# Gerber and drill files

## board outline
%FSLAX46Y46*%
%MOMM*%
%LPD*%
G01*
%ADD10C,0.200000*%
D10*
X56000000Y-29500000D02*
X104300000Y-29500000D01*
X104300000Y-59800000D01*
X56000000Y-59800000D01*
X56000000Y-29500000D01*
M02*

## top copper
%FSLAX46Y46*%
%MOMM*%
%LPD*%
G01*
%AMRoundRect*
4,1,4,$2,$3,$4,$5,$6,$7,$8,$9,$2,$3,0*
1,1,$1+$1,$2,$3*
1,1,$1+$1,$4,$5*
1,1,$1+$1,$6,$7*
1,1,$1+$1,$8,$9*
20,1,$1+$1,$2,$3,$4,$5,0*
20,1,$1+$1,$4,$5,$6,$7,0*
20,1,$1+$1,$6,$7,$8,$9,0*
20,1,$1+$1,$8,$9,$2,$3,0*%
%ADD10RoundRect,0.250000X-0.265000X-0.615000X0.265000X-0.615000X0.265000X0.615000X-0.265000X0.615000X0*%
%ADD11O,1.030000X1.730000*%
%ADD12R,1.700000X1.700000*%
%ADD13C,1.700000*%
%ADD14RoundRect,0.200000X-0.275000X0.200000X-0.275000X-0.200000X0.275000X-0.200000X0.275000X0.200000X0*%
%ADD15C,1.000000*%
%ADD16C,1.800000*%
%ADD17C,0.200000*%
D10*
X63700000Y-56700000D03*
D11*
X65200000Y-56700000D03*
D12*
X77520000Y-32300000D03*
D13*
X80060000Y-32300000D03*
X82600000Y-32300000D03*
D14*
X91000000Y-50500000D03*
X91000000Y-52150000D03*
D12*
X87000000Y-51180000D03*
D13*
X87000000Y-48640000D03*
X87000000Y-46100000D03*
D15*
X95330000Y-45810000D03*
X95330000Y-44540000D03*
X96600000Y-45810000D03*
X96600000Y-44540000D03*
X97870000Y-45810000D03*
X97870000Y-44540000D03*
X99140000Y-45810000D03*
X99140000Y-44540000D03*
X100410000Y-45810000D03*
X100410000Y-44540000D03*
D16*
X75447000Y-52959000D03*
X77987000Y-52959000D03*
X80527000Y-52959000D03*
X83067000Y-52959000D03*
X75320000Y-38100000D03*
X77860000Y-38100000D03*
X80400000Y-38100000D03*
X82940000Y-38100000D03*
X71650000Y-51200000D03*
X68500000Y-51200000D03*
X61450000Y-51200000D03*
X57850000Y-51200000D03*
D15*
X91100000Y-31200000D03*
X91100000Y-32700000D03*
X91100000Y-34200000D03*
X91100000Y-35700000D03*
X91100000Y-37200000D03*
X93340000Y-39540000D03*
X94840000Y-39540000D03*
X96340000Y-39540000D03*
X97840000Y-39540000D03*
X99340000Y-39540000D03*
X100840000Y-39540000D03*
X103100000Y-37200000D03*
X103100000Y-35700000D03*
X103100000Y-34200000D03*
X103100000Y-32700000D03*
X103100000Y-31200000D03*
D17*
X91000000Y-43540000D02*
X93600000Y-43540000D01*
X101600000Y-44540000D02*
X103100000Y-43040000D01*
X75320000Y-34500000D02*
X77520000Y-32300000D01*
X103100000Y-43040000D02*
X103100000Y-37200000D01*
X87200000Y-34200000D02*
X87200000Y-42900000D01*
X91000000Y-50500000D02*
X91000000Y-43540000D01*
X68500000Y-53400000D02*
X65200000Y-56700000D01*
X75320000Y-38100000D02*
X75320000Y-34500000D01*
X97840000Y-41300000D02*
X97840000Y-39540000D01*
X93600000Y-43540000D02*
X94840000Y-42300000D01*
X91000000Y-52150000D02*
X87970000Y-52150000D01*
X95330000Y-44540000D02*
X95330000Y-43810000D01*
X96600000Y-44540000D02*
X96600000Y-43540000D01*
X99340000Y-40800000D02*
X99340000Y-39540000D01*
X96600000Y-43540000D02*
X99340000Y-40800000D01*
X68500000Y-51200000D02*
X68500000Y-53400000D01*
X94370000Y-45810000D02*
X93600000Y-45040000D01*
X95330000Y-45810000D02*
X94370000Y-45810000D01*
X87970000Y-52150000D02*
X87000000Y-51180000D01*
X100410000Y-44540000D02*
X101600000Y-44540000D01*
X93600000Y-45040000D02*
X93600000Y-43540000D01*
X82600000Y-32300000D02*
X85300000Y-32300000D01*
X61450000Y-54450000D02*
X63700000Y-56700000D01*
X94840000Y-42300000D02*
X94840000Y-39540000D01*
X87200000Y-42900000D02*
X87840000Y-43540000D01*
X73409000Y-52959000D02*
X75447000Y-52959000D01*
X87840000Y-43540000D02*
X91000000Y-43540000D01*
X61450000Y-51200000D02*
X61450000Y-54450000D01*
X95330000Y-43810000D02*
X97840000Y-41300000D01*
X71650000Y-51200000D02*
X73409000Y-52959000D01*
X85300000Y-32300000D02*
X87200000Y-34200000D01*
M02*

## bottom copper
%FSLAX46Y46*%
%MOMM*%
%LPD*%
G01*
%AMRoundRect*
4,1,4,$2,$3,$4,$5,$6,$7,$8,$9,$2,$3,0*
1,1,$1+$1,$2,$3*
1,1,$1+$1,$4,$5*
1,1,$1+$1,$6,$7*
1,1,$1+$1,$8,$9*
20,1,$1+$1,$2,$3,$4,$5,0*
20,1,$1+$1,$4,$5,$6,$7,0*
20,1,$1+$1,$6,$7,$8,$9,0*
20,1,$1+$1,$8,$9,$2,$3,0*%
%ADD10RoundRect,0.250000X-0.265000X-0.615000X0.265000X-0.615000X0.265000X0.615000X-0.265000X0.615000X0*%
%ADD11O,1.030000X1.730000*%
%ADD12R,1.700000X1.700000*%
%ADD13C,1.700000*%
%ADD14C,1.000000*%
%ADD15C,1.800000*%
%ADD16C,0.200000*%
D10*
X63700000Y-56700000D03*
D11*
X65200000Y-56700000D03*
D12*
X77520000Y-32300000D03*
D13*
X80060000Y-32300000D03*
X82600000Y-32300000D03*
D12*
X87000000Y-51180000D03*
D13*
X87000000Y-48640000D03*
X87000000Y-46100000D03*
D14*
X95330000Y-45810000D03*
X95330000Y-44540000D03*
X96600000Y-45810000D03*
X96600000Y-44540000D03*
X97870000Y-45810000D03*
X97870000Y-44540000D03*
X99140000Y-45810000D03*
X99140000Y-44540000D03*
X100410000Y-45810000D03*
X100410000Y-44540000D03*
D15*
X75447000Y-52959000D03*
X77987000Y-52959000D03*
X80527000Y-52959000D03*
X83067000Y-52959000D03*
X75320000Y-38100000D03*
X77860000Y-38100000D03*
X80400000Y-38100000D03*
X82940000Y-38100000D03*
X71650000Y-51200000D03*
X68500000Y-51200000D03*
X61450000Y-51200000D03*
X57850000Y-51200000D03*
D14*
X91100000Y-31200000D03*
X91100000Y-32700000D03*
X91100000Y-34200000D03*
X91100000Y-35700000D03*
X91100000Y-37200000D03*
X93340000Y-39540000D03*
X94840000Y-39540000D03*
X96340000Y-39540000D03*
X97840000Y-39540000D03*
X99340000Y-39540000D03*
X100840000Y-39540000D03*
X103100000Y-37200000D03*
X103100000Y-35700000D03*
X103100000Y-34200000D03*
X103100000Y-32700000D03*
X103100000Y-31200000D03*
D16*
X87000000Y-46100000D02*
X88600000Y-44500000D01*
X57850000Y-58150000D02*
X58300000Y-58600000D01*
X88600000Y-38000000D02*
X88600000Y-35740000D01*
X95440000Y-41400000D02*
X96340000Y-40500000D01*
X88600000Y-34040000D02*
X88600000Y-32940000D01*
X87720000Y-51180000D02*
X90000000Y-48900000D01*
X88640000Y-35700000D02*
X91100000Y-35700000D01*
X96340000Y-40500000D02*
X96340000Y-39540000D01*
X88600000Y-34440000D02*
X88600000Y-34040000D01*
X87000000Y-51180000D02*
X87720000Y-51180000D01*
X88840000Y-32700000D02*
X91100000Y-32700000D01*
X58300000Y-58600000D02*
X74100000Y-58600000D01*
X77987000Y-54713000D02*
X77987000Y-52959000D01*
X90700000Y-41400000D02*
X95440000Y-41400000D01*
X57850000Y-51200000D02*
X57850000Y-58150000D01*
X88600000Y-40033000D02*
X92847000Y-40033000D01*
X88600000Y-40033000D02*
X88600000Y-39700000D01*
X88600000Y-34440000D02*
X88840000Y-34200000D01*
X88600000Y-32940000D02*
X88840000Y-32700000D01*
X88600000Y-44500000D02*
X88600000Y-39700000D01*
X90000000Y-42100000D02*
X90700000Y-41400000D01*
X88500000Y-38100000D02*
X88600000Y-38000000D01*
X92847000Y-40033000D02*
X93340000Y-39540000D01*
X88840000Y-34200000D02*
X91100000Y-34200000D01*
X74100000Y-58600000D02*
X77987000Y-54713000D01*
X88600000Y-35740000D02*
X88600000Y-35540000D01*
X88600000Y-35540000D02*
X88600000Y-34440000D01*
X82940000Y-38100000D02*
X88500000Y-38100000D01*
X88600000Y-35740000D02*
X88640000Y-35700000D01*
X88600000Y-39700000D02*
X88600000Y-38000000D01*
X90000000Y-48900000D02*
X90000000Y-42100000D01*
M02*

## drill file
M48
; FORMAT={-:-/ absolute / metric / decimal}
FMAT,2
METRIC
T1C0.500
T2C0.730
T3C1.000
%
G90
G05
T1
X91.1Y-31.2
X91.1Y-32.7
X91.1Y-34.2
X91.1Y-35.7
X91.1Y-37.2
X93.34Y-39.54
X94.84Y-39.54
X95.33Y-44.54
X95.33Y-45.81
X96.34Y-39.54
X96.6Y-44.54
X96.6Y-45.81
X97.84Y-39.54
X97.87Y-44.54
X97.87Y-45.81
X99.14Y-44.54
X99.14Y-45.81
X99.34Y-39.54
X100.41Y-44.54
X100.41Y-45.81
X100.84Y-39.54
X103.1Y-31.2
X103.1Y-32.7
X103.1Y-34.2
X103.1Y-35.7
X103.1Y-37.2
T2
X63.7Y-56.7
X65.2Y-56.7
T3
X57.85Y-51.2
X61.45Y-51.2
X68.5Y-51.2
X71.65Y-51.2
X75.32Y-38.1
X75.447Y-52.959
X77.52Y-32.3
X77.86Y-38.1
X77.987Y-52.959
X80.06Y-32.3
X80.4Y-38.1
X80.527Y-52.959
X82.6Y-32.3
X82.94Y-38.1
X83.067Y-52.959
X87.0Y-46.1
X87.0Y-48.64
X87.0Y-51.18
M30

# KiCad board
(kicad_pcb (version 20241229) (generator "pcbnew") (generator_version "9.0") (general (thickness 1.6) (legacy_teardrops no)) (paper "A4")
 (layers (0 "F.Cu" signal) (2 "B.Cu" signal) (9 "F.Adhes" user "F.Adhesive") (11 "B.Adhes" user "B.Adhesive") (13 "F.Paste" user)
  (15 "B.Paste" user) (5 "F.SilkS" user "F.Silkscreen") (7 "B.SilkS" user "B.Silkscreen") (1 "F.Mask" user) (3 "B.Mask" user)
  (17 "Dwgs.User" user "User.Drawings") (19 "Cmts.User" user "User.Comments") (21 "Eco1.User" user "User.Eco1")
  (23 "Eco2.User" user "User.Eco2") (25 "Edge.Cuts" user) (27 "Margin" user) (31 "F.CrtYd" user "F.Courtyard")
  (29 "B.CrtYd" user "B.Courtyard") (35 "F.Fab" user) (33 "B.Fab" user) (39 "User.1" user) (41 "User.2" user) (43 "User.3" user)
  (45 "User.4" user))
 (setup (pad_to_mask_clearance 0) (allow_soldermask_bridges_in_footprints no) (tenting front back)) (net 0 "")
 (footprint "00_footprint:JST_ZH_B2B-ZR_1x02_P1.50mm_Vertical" (layer "F.Cu") (at 63.7 56.7)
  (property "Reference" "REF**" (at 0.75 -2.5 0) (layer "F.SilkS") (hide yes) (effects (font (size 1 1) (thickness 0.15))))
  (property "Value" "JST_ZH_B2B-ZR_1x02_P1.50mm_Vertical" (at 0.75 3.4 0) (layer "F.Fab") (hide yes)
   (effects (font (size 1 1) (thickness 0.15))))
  (pad "1" thru_hole roundrect (at 0 0) (size 1.03 1.73) (drill 0.73) (layers "*.Cu" "*.Mask") (remove_unused_layers no)
   (roundrect_rratio 0.242718))
  (pad "2" thru_hole oval (at 1.5 0) (size 1.03 1.73) (drill 0.73) (layers "*.Cu" "*.Mask") (remove_unused_layers no)))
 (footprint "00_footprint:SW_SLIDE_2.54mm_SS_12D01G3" (layer "F.Cu") (at 77.52 32.3 90)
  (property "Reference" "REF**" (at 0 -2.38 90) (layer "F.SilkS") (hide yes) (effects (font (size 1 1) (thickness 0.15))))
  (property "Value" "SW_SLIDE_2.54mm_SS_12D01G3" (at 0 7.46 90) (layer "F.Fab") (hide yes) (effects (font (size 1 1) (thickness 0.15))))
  (pad "1" thru_hole rect (at 0 0 90) (size 1.7 1.7) (drill 1) (layers "*.Cu" "*.Mask") (remove_unused_layers no))
  (pad "2" thru_hole circle (at 0 2.54 90) (size 1.7 1.7) (drill 1) (layers "*.Cu" "*.Mask") (remove_unused_layers no))
  (pad "3" thru_hole circle (at 0 5.08 90) (size 1.7 1.7) (drill 1) (layers "*.Cu" "*.Mask") (remove_unused_layers no)))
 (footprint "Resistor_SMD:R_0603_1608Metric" (layer "F.Cu") (at 91 51.325 -90)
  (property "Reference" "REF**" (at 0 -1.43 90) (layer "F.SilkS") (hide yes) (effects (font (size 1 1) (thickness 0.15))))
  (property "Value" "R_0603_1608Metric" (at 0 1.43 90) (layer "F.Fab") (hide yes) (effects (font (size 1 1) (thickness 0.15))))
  (pad "1" smd roundrect (at -0.825 0 270) (size 0.8 0.95) (layers "F.Cu" "F.Mask" "F.Paste") (roundrect_rratio 0.25))
  (pad "2" smd roundrect (at 0.825 0 270) (size 0.8 0.95) (layers "F.Cu" "F.Mask" "F.Paste") (roundrect_rratio 0.25)))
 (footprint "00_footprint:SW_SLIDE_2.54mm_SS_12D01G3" (layer "F.Cu") (at 87 51.18 180)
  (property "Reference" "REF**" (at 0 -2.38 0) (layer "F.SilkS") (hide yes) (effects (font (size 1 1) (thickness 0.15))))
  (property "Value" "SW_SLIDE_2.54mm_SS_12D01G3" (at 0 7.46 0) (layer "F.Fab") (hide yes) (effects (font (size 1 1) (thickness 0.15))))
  (pad "1" thru_hole rect (at 0 0 180) (size 1.7 1.7) (drill 1) (layers "*.Cu" "*.Mask") (remove_unused_layers no))
  (pad "2" thru_hole circle (at 0 2.54 180) (size 1.7 1.7) (drill 1) (layers "*.Cu" "*.Mask") (remove_unused_layers no))
  (pad "3" thru_hole circle (at 0 5.08 180) (size 1.7 1.7) (drill 1) (layers "*.Cu" "*.Mask") (remove_unused_layers no)))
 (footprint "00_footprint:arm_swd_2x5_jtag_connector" (layer "F.Cu") (at 97.87 45.81 180)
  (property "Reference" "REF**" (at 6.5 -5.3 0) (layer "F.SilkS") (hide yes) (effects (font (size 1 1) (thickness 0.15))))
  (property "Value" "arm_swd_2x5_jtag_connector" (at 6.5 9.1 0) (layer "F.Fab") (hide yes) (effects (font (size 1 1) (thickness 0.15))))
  (pad "1" thru_hole circle (at 2.54 0 270) (size 1 1) (drill 0.5) (layers "*.Cu" "*.Mask") (remove_unused_layers no))
  (pad "2" thru_hole circle (at 2.54 1.27 270) (size 1 1) (drill 0.5) (layers "*.Cu" "*.Mask") (remove_unused_layers no))
  (pad "3" thru_hole circle (at 1.27 0 270) (size 1 1) (drill 0.5) (layers "*.Cu" "*.Mask") (remove_unused_layers no))
  (pad "4" thru_hole circle (at 1.27 1.27 270) (size 1 1) (drill 0.5) (layers "*.Cu" "*.Mask") (remove_unused_layers no))
  (pad "5" thru_hole circle (at 0 0 270) (size 1 1) (drill 0.5) (layers "*.Cu" "*.Mask") (remove_unused_layers no))
  (pad "6" thru_hole circle (at 0 1.27 270) (size 1 1) (drill 0.5) (layers "*.Cu" "*.Mask") (remove_unused_layers no))
  (pad "7" thru_hole circle (at -1.27 0 270) (size 1 1) (drill 0.5) (layers "*.Cu" "*.Mask") (remove_unused_layers no))
  (pad "8" thru_hole circle (at -1.27 1.27 270) (size 1 1) (drill 0.5) (layers "*.Cu" "*.Mask") (remove_unused_layers no))
  (pad "9" thru_hole circle (at -2.54 0 270) (size 1 1) (drill 0.5) (layers "*.Cu" "*.Mask") (remove_unused_layers no))
  (pad "10" thru_hole circle (at -2.54 1.27 270) (size 1 1) (drill 0.5) (layers "*.Cu" "*.Mask") (remove_unused_layers no)))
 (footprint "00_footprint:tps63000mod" (layer "F.Cu") (at 79.257 45.593 90)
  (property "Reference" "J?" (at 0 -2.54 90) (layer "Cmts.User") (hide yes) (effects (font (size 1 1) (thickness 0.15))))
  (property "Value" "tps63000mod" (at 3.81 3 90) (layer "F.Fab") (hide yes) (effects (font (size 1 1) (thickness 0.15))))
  (pad "1" thru_hole circle (at -7.366 -3.81 90) (size 1.8 1.8) (drill 1) (layers "*.Cu" "*.Mask") (remove_unused_layers no))
  (pad "2" thru_hole circle (at -7.366 -1.27 90) (size 1.8 1.8) (drill 1) (layers "*.Cu" "*.Mask") (remove_unused_layers no))
  (pad "3" thru_hole circle (at -7.366 1.27 90) (size 1.8 1.8) (drill 1) (layers "*.Cu" "*.Mask") (remove_unused_layers no))
  (pad "4" thru_hole circle (at -7.366 3.81 90) (size 1.8 1.8) (drill 1) (layers "*.Cu" "*.Mask") (remove_unused_layers no))
  (pad "5" thru_hole circle (at 7.493 -3.937 90) (size 1.8 1.8) (drill 1) (layers "*.Cu" "*.Mask") (remove_unused_layers no))
  (pad "6" thru_hole circle (at 7.493 -1.397 90) (size 1.8 1.8) (drill 1) (layers "*.Cu" "*.Mask") (remove_unused_layers no))
  (pad "7" thru_hole circle (at 7.493 1.143 90) (size 1.8 1.8) (drill 1) (layers "*.Cu" "*.Mask") (remove_unused_layers no))
  (pad "8" thru_hole circle (at 7.493 3.683 90) (size 1.8 1.8) (drill 1) (layers "*.Cu" "*.Mask") (remove_unused_layers no)))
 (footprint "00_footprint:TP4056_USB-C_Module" (layer "F.Cu") (at 64.4 42 -90)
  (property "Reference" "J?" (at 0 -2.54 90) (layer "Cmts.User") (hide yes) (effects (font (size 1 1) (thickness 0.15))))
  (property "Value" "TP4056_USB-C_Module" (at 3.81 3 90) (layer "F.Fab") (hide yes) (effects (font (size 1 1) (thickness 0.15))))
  (pad "1" thru_hole circle (at 9.2 -7.25 270) (size 1.8 1.8) (drill 1) (layers "*.Cu" "*.Mask") (remove_unused_layers no))
  (pad "2" thru_hole circle (at 9.2 -4.1 270) (size 1.8 1.8) (drill 1) (layers "*.Cu" "*.Mask") (remove_unused_layers no))
  (pad "3" thru_hole circle (at 9.2 2.95 270) (size 1.8 1.8) (drill 1) (layers "*.Cu" "*.Mask") (remove_unused_layers no))
  (pad "4" thru_hole circle (at 9.2 6.55 270) (size 1.8 1.8) (drill 1) (layers "*.Cu" "*.Mask") (remove_unused_layers no)))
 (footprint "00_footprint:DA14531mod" (layer "F.Cu") (at 97.1 34.54)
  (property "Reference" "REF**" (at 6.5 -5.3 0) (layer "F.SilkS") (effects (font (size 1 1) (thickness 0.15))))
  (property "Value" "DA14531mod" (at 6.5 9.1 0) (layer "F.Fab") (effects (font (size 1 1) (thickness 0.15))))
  (pad "J1" thru_hole circle (at -6 -3.34 90) (size 1 1) (drill 0.5) (layers "*.Cu" "*.Mask") (remove_unused_layers no))
  (pad "J2" thru_hole circle (at -6 -1.84 90) (size 1 1) (drill 0.5) (layers "*.Cu" "*.Mask") (remove_unused_layers no))
  (pad "J3" thru_hole circle (at -6 -0.34 90) (size 1 1) (drill 0.5) (layers "*.Cu" "*.Mask") (remove_unused_layers no))
  (pad "J4" thru_hole circle (at -6 1.16 90) (size 1 1) (drill 0.5) (layers "*.Cu" "*.Mask") (remove_unused_layers no))
  (pad "J5" thru_hole circle (at -6 2.66 90) (size 1 1) (drill 0.5) (layers "*.Cu" "*.Mask") (remove_unused_layers no))
  (pad "J6" thru_hole circle (at -3.76 5 90) (size 1 1) (drill 0.5) (layers "*.Cu" "*.Mask") (remove_unused_layers no))
  (pad "J7" thru_hole circle (at -2.26 5 90) (size 1 1) (drill 0.5) (layers "*.Cu" "*.Mask") (remove_unused_layers no))
  (pad "J8" thru_hole circle (at -0.76 5 90) (size 1 1) (drill 0.5) (layers "*.Cu" "*.Mask") (remove_unused_layers no))
  (pad "J9" thru_hole circle (at 0.74 5 90) (size 1 1) (drill 0.5) (layers "*.Cu" "*.Mask") (remove_unused_layers no))
  (pad "J10" thru_hole circle (at 2.24 5 90) (size 1 1) (drill 0.5) (layers "*.Cu" "*.Mask") (remove_unused_layers no))
  (pad "J11" thru_hole circle (at 3.74 5 90) (size 1 1) (drill 0.5) (layers "*.Cu" "*.Mask") (remove_unused_layers no))
  (pad "J12" thru_hole circle (at 6 2.66 90) (size 1 1) (drill 0.5) (layers "*.Cu" "*.Mask") (remove_unused_layers no))
  (pad "J13" thru_hole circle (at 6 1.16 90) (size 1 1) (drill 0.5) (layers "*.Cu" "*.Mask") (remove_unused_layers no))
  (pad "J14" thru_hole circle (at 6 -0.34 90) (size 1 1) (drill 0.5) (layers "*.Cu" "*.Mask") (remove_unused_layers no))
  (pad "J15" thru_hole circle (at 6 -1.84 90) (size 1 1) (drill 0.5) (layers "*.Cu" "*.Mask") (remove_unused_layers no))
  (pad "J16" thru_hole circle (at 6 -3.34 90) (size 1 1) (drill 0.5) (layers "*.Cu" "*.Mask") (remove_unused_layers no)))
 (gr_rect (start 56 29.5) (end 104.3 59.8) (stroke (width 0.2) (type solid)) (fill no) (layer "Edge.Cuts"))
 (segment (start 91 43.54) (end 93.6 43.54) (width 0.2) (layer "F.Cu") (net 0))
 (segment (start 101.6 44.54) (end 103.1 43.04) (width 0.2) (layer "F.Cu") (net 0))
 (segment (start 75.32 34.5) (end 77.52 32.3) (width 0.2) (layer "F.Cu") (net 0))
 (segment (start 103.1 43.04) (end 103.1 37.2) (width 0.2) (layer "F.Cu") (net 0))
 (segment (start 87.2 34.2) (end 87.2 42.9) (width 0.2) (layer "F.Cu") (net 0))
 (segment (start 91 50.5) (end 91 43.54) (width 0.2) (layer "F.Cu") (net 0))
 (segment (start 68.5 53.4) (end 65.2 56.7) (width 0.2) (layer "F.Cu") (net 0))
 (segment (start 75.32 38.1) (end 75.32 34.5) (width 0.2) (layer "F.Cu") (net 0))
 (segment (start 97.84 41.3) (end 97.84 39.54) (width 0.2) (layer "F.Cu") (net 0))
 (segment (start 93.6 43.54) (end 94.84 42.3) (width 0.2) (layer "F.Cu") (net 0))
 (segment (start 91 52.15) (end 87.97 52.15) (width 0.2) (layer "F.Cu") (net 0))
 (segment (start 95.33 44.54) (end 95.33 43.81) (width 0.2) (layer "F.Cu") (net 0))
 (segment (start 96.6 44.54) (end 96.6 43.54) (width 0.2) (layer "F.Cu") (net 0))
 (segment (start 99.34 40.8) (end 99.34 39.54) (width 0.2) (layer "F.Cu") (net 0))
 (segment (start 96.6 43.54) (end 99.34 40.8) (width 0.2) (layer "F.Cu") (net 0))
 (segment (start 68.5 51.2) (end 68.5 53.4) (width 0.2) (layer "F.Cu") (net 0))
 (segment (start 94.37 45.81) (end 93.6 45.04) (width 0.2) (layer "F.Cu") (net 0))
 (segment (start 95.33 45.81) (end 94.37 45.81) (width 0.2) (layer "F.Cu") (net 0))
 (segment (start 87.97 52.15) (end 87 51.18) (width 0.2) (layer "F.Cu") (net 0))
 (segment (start 100.41 44.54) (end 101.6 44.54) (width 0.2) (layer "F.Cu") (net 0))
 (segment (start 93.6 45.04) (end 93.6 43.54) (width 0.2) (layer "F.Cu") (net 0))
 (segment (start 82.6 32.3) (end 85.3 32.3) (width 0.2) (layer "F.Cu") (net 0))
 (segment (start 61.45 54.45) (end 63.7 56.7) (width 0.2) (layer "F.Cu") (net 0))
 (segment (start 94.84 42.3) (end 94.84 39.54) (width 0.2) (layer "F.Cu") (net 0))
 (segment (start 87.2 42.9) (end 87.84 43.54) (width 0.2) (layer "F.Cu") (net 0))
 (segment (start 73.409 52.959) (end 75.447 52.959) (width 0.2) (layer "F.Cu") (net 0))
 (segment (start 87.84 43.54) (end 91 43.54) (width 0.2) (layer "F.Cu") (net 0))
 (segment (start 61.45 51.2) (end 61.45 54.45) (width 0.2) (layer "F.Cu") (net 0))
 (segment (start 95.33 43.81) (end 97.84 41.3) (width 0.2) (layer "F.Cu") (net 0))
 (segment (start 71.65 51.2) (end 73.409 52.959) (width 0.2) (layer "F.Cu") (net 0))
 (segment (start 85.3 32.3) (end 87.2 34.2) (width 0.2) (layer "F.Cu") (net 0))
 (segment (start 87 46.1) (end 88.6 44.5) (width 0.2) (layer "B.Cu") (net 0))
 (segment (start 57.85 58.15) (end 58.3 58.6) (width 0.2) (layer "B.Cu") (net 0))
 (segment (start 88.6 38) (end 88.6 35.74) (width 0.2) (layer "B.Cu") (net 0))
 (segment (start 95.44 41.4) (end 96.34 40.5) (width 0.2) (layer "B.Cu") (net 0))
 (segment (start 88.6 34.04) (end 88.6 32.94) (width 0.2) (layer "B.Cu") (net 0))
 (segment (start 87.72 51.18) (end 90 48.9) (width 0.2) (layer "B.Cu") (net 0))
 (segment (start 88.64 35.7) (end 91.1 35.7) (width 0.2) (layer "B.Cu") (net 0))
 (segment (start 96.34 40.5) (end 96.34 39.54) (width 0.2) (layer "B.Cu") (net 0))
 (segment (start 88.6 34.44) (end 88.6 34.04) (width 0.2) (layer "B.Cu") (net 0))
 (segment (start 87 51.18) (end 87.72 51.18) (width 0.2) (layer "B.Cu") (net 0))
 (segment (start 88.84 32.7) (end 91.1 32.7) (width 0.2) (layer "B.Cu") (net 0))
 (segment (start 58.3 58.6) (end 74.1 58.6) (width 0.2) (layer "B.Cu") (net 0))
 (segment (start 77.987 54.713) (end 77.987 52.959) (width 0.2) (layer "B.Cu") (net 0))
 (segment (start 90.7 41.4) (end 95.44 41.4) (width 0.2) (layer "B.Cu") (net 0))
 (segment (start 57.85 51.2) (end 57.85 58.15) (width 0.2) (layer "B.Cu") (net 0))
 (segment (start 88.6 40.033) (end 92.847 40.033) (width 0.2) (layer "B.Cu") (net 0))
 (segment (start 88.6 40.033) (end 88.6 39.7) (width 0.2) (layer "B.Cu") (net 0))
 (segment (start 88.6 34.44) (end 88.84 34.2) (width 0.2) (layer "B.Cu") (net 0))
 (segment (start 88.6 32.94) (end 88.84 32.7) (width 0.2) (layer "B.Cu") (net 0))
 (segment (start 88.6 44.5) (end 88.6 39.7) (width 0.2) (layer "B.Cu") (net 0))
 (segment (start 90 42.1) (end 90.7 41.4) (width 0.2) (layer "B.Cu") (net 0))
 (segment (start 88.5 38.1) (end 88.6 38) (width 0.2) (layer "B.Cu") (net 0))
 (segment (start 92.847 40.033) (end 93.34 39.54) (width 0.2) (layer "B.Cu") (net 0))
 (segment (start 88.84 34.2) (end 91.1 34.2) (width 0.2) (layer "B.Cu") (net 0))
 (segment (start 74.1 58.6) (end 77.987 54.713) (width 0.2) (layer "B.Cu") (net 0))
 (segment (start 88.6 35.74) (end 88.6 35.54) (width 0.2) (layer "B.Cu") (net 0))
 (segment (start 88.6 35.54) (end 88.6 34.44) (width 0.2) (layer "B.Cu") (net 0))
 (segment (start 82.94 38.1) (end 88.5 38.1) (width 0.2) (layer "B.Cu") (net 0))
 (segment (start 88.6 35.74) (end 88.64 35.7) (width 0.2) (layer "B.Cu") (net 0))
 (segment (start 88.6 39.7) (end 88.6 38) (width 0.2) (layer "B.Cu") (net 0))
 (segment (start 90 48.9) (end 90 42.1) (width 0.2) (layer "B.Cu") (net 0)))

